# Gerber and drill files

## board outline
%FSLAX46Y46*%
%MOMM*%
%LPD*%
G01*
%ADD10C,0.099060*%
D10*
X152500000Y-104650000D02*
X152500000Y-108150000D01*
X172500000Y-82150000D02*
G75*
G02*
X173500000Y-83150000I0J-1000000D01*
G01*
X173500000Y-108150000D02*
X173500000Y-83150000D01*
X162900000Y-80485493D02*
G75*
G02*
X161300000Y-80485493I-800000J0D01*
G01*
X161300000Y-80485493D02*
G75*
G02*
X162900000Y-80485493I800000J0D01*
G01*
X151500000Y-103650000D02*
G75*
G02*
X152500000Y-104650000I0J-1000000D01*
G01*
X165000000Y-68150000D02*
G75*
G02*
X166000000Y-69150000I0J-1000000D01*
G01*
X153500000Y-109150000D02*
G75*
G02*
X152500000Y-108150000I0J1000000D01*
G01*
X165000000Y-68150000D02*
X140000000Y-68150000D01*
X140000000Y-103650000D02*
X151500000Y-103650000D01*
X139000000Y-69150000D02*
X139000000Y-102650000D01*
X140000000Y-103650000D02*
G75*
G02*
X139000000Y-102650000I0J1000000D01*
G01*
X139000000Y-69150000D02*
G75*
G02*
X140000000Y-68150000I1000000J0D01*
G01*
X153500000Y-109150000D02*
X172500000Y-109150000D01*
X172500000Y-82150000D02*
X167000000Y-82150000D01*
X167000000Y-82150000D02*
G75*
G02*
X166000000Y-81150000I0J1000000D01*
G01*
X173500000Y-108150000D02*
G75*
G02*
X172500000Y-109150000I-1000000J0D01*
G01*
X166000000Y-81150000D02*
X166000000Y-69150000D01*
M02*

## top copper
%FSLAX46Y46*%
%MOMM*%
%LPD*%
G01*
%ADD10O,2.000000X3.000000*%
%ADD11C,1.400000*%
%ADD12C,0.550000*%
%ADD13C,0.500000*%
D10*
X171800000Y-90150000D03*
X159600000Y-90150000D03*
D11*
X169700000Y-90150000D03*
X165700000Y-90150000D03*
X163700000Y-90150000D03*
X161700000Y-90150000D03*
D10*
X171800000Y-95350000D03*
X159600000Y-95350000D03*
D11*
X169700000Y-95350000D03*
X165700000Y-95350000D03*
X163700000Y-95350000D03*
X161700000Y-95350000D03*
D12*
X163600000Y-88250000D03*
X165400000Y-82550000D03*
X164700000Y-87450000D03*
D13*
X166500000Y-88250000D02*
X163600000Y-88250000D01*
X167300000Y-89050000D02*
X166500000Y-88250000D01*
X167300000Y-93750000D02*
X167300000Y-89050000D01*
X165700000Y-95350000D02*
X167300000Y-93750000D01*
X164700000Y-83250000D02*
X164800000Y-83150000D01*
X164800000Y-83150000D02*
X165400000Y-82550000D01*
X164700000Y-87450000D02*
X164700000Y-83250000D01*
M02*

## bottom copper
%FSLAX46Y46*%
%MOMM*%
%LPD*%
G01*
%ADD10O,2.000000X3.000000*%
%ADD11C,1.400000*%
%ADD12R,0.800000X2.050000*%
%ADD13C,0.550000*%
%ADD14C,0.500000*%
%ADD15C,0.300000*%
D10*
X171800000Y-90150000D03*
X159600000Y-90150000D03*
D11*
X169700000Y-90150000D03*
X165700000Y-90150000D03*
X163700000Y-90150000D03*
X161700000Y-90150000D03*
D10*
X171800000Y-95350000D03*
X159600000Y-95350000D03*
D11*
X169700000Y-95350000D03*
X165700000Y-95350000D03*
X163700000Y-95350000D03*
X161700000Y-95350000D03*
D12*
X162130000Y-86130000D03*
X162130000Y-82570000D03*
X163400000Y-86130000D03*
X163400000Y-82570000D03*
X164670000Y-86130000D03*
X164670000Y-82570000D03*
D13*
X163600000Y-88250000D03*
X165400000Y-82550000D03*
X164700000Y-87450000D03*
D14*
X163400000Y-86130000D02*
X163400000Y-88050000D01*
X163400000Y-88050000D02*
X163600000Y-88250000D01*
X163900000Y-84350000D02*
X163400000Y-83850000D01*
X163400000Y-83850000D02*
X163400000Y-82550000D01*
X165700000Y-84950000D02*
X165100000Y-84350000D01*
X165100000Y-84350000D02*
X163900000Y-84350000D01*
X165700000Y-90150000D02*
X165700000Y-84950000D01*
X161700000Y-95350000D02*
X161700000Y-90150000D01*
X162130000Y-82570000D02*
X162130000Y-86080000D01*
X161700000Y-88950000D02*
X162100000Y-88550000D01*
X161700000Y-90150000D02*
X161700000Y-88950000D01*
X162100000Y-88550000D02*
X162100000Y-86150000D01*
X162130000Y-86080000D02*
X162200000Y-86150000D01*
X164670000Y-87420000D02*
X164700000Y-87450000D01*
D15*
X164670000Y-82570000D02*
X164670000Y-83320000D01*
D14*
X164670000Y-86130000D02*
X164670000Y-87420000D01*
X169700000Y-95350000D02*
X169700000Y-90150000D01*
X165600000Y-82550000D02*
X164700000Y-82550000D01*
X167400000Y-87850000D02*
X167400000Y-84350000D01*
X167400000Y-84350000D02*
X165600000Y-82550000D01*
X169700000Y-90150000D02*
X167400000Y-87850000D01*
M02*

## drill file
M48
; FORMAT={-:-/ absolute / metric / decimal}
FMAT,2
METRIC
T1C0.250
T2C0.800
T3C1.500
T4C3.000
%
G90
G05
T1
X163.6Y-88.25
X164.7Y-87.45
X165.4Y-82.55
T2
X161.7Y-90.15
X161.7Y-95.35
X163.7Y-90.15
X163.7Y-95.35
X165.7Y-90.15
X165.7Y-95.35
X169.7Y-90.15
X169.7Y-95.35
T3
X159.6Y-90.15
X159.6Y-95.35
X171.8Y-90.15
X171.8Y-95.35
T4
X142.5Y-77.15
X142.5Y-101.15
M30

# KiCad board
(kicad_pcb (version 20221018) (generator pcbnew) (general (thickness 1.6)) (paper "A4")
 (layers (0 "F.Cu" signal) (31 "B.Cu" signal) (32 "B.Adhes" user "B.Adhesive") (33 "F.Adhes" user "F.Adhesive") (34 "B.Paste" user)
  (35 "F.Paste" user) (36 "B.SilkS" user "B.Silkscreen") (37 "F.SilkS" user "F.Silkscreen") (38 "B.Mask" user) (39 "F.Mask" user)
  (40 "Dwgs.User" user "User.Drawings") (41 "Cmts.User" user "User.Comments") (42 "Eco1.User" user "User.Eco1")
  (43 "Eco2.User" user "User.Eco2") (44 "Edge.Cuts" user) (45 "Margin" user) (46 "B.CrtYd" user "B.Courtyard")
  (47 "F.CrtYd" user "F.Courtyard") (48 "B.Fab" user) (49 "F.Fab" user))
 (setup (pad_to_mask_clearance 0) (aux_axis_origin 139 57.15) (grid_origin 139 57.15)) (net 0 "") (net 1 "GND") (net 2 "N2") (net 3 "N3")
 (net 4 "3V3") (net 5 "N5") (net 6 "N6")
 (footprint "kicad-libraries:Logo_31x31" (layer "F.Cu") (at 168.5 104.65)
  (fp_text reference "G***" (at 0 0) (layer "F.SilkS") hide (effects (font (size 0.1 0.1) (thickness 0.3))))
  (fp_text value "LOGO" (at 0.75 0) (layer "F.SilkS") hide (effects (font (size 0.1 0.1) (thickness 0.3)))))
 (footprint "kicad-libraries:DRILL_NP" (layer "F.Cu") (at 142.5 101.15)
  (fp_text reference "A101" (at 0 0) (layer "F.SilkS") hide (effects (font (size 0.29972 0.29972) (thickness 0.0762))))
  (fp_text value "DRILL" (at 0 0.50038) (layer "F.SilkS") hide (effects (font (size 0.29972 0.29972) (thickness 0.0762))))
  (pad "" np_thru_hole circle (at 0 0) (size 2.99974 2.99974) (drill 2.99974) (layers "*.Cu" "*.Mask" "F.SilkS") (clearance 0.89916)))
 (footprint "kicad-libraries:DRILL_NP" (layer "F.Cu") (at 142.5 77.15)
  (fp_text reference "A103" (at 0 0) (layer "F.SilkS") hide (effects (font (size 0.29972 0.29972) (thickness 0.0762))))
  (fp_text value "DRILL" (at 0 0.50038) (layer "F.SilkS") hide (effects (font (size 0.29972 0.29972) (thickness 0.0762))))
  (pad "" np_thru_hole circle (at 0 0) (size 2.99974 2.99974) (drill 2.99974) (layers "*.Cu" "*.Mask" "F.SilkS") (clearance 0.89916)))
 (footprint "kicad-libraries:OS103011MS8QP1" (layer "F.Cu") (at 165.7 90.15 180)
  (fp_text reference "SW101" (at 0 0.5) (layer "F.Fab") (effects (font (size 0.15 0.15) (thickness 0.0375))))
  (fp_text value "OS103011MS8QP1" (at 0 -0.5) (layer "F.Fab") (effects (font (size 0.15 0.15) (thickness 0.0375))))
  (pad "" thru_hole oval (at -6.1 0 180) (size 2 3) (drill 1.5) (layers "*.Cu" "*.Mask"))
  (pad "" thru_hole oval (at 6.1 0 180) (size 2 3) (drill 1.5) (layers "*.Cu" "*.Mask"))
  (pad "1" thru_hole circle (at -4 0 180) (size 1.4 1.4) (drill 0.8) (layers "*.Cu" "*.Mask") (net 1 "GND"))
  (pad "2" thru_hole circle (at 0 0 180) (size 1.4 1.4) (drill 0.8) (layers "*.Cu" "*.Mask") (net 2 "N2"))
  (pad "3" thru_hole circle (at 2 0 180) (size 1.4 1.4) (drill 0.8) (layers "*.Cu" "*.Mask") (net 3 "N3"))
  (pad "4" thru_hole circle (at 4 0 180) (size 1.4 1.4) (drill 0.8) (layers "*.Cu" "*.Mask") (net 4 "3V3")))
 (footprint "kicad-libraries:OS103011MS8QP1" (layer "F.Cu") (at 165.7 95.35 180)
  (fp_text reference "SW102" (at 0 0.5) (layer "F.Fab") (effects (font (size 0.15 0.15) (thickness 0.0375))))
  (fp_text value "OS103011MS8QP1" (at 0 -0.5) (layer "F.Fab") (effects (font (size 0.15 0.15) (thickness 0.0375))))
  (pad "" thru_hole oval (at -6.1 0 180) (size 2 3) (drill 1.5) (layers "*.Cu" "*.Mask"))
  (pad "" thru_hole oval (at 6.1 0 180) (size 2 3) (drill 1.5) (layers "*.Cu" "*.Mask"))
  (pad "1" thru_hole circle (at -4 0 180) (size 1.4 1.4) (drill 0.8) (layers "*.Cu" "*.Mask") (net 1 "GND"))
  (pad "2" thru_hole circle (at 0 0 180) (size 1.4 1.4) (drill 0.8) (layers "*.Cu" "*.Mask") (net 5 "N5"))
  (pad "3" thru_hole circle (at 2 0 180) (size 1.4 1.4) (drill 0.8) (layers "*.Cu" "*.Mask") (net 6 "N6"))
  (pad "4" thru_hole circle (at 4 0 180) (size 1.4 1.4) (drill 0.8) (layers "*.Cu" "*.Mask") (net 4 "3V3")))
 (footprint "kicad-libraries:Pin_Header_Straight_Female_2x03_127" (layer "B.Cu") (at 163.4 84.35)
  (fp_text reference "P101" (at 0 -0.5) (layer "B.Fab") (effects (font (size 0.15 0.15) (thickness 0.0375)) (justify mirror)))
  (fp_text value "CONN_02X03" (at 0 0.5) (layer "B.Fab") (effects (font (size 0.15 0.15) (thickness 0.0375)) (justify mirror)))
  (pad "1" smd rect (at -1.27 1.78) (size 0.8 2.05) (layers "B.Cu" "B.Paste" "B.Mask") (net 4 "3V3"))
  (pad "2" smd rect (at -1.27 -1.78) (size 0.8 2.05) (layers "B.Cu" "B.Paste" "B.Mask") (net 4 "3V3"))
  (pad "3" smd rect (at 0 1.78) (size 0.8 2.05) (layers "B.Cu" "B.Paste" "B.Mask") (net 5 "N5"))
  (pad "4" smd rect (at 0 -1.78) (size 0.8 2.05) (layers "B.Cu" "B.Paste" "B.Mask") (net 2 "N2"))
  (pad "5" smd rect (at 1.27 1.78) (size 0.8 2.05) (layers "B.Cu" "B.Paste" "B.Mask") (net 1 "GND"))
  (pad "6" smd rect (at 1.27 -1.78) (size 0.8 2.05) (layers "B.Cu" "B.Paste" "B.Mask") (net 1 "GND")))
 (gr_line (start 152.5 104.65) (end 152.5 108.15) (stroke (width 0.09906) (type solid)) (layer "Edge.Cuts"))
 (gr_arc (start 172.5 82.15) (mid 173.207107 82.442893) (end 173.5 83.15) (stroke (width 0.09906) (type solid)) (layer "Edge.Cuts"))
 (gr_line (start 173.5 108.15) (end 173.5 83.15) (stroke (width 0.09906) (type solid)) (layer "Edge.Cuts"))
 (gr_circle (center 162.1 80.485493) (end 162.9 80.485493) (stroke (width 0.09906) (type solid)) (fill none) (layer "Edge.Cuts"))
 (gr_arc (start 151.5 103.65) (mid 152.207107 103.942893) (end 152.5 104.65) (stroke (width 0.09906) (type solid)) (layer "Edge.Cuts"))
 (gr_arc (start 165 68.15) (mid 165.707107 68.442893) (end 166 69.15) (stroke (width 0.09906) (type solid)) (layer "Edge.Cuts"))
 (gr_arc (start 153.5 109.15) (mid 152.792893 108.857107) (end 152.5 108.15) (stroke (width 0.09906) (type solid)) (layer "Edge.Cuts"))
 (gr_line (start 165 68.15) (end 140 68.15) (stroke (width 0.09906) (type solid)) (layer "Edge.Cuts"))
 (gr_line (start 140 103.65) (end 151.5 103.65) (stroke (width 0.09906) (type solid)) (layer "Edge.Cuts"))
 (gr_line (start 139 69.15) (end 139 102.65) (stroke (width 0.09906) (type solid)) (layer "Edge.Cuts"))
 (gr_arc (start 140 103.65) (mid 139.292893 103.357107) (end 139 102.65) (stroke (width 0.09906) (type solid)) (layer "Edge.Cuts"))
 (gr_arc (start 139 69.15) (mid 139.292893 68.442893) (end 140 68.15) (stroke (width 0.09906) (type solid)) (layer "Edge.Cuts"))
 (gr_line (start 153.5 109.15) (end 172.5 109.15) (stroke (width 0.09906) (type solid)) (layer "Edge.Cuts"))
 (gr_line (start 172.5 82.15) (end 167 82.15) (stroke (width 0.09906) (type solid)) (layer "Edge.Cuts"))
 (gr_arc (start 167 82.15) (mid 166.292893 81.857107) (end 166 81.15) (stroke (width 0.09906) (type solid)) (layer "Edge.Cuts"))
 (gr_arc (start 173.5 108.15) (mid 173.207107 108.857107) (end 172.5 109.15) (stroke (width 0.09906) (type solid)) (layer "Edge.Cuts"))
 (gr_line (start 166 81.15) (end 166 69.15) (stroke (width 0.09906) (type solid)) (layer "Edge.Cuts"))
 (segment (start 166.5 88.25) (end 163.6 88.25) (width 0.5) (layer "F.Cu") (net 5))
 (segment (start 167.3 89.05) (end 166.5 88.25) (width 0.5) (layer "F.Cu") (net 5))
 (segment (start 167.3 93.75) (end 167.3 89.05) (width 0.5) (layer "F.Cu") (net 5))
 (segment (start 165.7 95.35) (end 167.3 93.75) (width 0.5) (layer "F.Cu") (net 5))
 (via (at 163.6 88.25) (size 0.55) (drill 0.25) (layers "F.Cu" "B.Cu") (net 5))
 (segment (start 163.4 86.13) (end 163.4 88.05) (width 0.5) (layer "B.Cu") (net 5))
 (segment (start 163.4 88.05) (end 163.6 88.25) (width 0.5) (layer "B.Cu") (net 5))
 (segment (start 163.9 84.35) (end 163.4 83.85) (width 0.5) (layer "B.Cu") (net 2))
 (segment (start 163.4 83.85) (end 163.4 82.55) (width 0.5) (layer "B.Cu") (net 2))
 (segment (start 165.7 84.95) (end 165.1 84.35) (width 0.5) (layer "B.Cu") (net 2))
 (segment (start 165.1 84.35) (end 163.9 84.35) (width 0.5) (layer "B.Cu") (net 2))
 (segment (start 165.7 90.15) (end 165.7 84.95) (width 0.5) (layer "B.Cu") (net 2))
 (segment (start 161.7 95.35) (end 161.7 90.15) (width 0.5) (layer "B.Cu") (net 4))
 (segment (start 162.13 82.57) (end 162.13 86.08) (width 0.5) (layer "B.Cu") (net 4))
 (segment (start 161.7 88.95) (end 162.1 88.55) (width 0.5) (layer "B.Cu") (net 4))
 (segment (start 161.7 90.15) (end 161.7 88.95) (width 0.5) (layer "B.Cu") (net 4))
 (segment (start 162.1 88.55) (end 162.1 86.15) (width 0.5) (layer "B.Cu") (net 4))
 (segment (start 162.13 86.08) (end 162.2 86.15) (width 0.5) (layer "B.Cu") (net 4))
 (segment (start 164.7 83.25) (end 164.8 83.15) (width 0.5) (layer "F.Cu") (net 1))
 (segment (start 164.8 83.15) (end 165.4 82.55) (width 0.5) (layer "F.Cu") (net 1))
 (segment (start 164.7 87.45) (end 164.7 83.25) (width 0.5) (layer "F.Cu") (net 1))
 (via (at 165.4 82.55) (size 0.55) (drill 0.25) (layers "F.Cu" "B.Cu") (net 1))
 (via (at 164.7 87.45) (size 0.55) (drill 0.25) (layers "F.Cu" "B.Cu") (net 1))
 (segment (start 164.67 87.42) (end 164.7 87.45) (width 0.5) (layer "B.Cu") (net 1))
 (segment (start 164.67 82.57) (end 164.67 83.32) (width 0.3) (layer "B.Cu") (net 1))
 (segment (start 164.67 86.13) (end 164.67 87.42) (width 0.5) (layer "B.Cu") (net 1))
 (segment (start 169.7 95.35) (end 169.7 90.15) (width 0.5) (layer "B.Cu") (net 1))
 (segment (start 165.6 82.55) (end 164.7 82.55) (width 0.5) (layer "B.Cu") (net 1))
 (segment (start 167.4 87.85) (end 167.4 84.35) (width 0.5) (layer "B.Cu") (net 1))
 (segment (start 167.4 84.35) (end 165.6 82.55) (width 0.5) (layer "B.Cu") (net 1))
 (segment (start 169.7 90.15) (end 167.4 87.85) (width 0.5) (layer "B.Cu") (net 1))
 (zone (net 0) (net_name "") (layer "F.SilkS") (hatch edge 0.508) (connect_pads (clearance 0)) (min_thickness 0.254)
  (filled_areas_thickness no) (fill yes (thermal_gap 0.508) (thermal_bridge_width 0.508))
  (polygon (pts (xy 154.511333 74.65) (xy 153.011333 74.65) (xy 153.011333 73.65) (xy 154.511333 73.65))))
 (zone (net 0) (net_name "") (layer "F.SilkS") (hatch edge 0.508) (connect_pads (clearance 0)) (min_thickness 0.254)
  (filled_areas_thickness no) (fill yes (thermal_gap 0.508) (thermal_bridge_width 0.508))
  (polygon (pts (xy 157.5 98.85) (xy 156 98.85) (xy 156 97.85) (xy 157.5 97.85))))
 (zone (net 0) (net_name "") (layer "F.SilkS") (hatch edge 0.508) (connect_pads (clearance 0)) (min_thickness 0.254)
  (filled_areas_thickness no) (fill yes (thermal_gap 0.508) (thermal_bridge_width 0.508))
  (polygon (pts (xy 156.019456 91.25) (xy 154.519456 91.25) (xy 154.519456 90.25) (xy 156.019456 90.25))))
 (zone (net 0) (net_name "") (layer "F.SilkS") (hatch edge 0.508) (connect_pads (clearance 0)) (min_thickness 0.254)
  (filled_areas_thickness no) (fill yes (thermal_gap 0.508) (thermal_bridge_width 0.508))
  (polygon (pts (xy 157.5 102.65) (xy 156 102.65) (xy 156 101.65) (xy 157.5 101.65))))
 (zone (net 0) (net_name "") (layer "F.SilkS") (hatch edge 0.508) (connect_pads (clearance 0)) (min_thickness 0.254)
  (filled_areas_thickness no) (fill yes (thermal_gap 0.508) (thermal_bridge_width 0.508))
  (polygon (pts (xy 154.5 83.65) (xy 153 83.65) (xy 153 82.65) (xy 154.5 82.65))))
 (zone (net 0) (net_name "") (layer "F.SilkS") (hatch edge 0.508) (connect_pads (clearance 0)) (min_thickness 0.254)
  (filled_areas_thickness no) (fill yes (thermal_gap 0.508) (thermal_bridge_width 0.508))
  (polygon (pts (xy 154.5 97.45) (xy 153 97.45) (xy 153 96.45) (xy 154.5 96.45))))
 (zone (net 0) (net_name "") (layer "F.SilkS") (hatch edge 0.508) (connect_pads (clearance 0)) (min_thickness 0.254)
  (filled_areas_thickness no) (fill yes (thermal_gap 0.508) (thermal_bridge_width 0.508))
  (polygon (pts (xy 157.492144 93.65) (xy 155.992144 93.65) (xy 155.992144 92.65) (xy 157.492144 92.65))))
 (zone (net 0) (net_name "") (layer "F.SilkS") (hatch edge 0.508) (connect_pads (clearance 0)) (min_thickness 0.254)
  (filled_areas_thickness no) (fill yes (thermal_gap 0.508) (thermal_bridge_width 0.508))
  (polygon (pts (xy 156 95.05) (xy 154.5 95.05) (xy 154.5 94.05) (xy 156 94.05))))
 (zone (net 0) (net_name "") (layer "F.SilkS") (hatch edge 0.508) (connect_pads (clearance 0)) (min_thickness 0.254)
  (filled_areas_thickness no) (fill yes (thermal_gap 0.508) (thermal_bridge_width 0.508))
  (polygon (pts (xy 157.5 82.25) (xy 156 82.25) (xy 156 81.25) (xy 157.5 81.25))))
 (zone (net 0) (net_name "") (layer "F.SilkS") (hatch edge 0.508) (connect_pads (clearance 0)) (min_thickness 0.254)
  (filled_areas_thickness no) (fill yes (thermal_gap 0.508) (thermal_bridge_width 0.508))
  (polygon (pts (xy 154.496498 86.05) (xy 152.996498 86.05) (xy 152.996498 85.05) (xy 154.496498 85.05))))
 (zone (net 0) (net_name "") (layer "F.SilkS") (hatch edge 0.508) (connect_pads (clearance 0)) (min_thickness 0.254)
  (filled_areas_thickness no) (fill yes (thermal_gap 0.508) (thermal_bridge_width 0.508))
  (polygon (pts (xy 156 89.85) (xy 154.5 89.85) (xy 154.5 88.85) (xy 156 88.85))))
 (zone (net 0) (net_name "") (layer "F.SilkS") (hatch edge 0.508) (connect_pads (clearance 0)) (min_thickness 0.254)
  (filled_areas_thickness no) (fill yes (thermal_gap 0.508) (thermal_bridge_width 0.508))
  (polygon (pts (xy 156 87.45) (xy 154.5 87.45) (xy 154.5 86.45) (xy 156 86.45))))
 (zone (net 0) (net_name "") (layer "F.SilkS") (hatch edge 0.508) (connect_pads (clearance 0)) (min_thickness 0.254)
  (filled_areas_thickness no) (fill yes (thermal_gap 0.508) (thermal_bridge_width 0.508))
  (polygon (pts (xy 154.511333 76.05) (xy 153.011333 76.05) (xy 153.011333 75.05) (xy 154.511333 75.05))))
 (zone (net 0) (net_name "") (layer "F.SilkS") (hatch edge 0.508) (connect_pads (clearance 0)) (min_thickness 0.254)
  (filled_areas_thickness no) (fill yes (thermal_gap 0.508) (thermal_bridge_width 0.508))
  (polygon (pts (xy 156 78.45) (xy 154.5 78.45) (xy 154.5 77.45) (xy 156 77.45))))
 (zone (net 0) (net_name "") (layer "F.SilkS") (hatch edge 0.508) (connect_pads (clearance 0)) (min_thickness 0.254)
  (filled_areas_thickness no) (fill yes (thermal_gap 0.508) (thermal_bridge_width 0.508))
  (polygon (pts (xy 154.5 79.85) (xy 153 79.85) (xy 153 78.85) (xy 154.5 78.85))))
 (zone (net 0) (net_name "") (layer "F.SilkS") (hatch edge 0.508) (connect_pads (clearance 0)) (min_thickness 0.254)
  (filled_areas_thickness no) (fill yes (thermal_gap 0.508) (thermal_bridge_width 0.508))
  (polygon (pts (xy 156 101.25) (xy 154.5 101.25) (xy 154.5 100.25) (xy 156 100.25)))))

